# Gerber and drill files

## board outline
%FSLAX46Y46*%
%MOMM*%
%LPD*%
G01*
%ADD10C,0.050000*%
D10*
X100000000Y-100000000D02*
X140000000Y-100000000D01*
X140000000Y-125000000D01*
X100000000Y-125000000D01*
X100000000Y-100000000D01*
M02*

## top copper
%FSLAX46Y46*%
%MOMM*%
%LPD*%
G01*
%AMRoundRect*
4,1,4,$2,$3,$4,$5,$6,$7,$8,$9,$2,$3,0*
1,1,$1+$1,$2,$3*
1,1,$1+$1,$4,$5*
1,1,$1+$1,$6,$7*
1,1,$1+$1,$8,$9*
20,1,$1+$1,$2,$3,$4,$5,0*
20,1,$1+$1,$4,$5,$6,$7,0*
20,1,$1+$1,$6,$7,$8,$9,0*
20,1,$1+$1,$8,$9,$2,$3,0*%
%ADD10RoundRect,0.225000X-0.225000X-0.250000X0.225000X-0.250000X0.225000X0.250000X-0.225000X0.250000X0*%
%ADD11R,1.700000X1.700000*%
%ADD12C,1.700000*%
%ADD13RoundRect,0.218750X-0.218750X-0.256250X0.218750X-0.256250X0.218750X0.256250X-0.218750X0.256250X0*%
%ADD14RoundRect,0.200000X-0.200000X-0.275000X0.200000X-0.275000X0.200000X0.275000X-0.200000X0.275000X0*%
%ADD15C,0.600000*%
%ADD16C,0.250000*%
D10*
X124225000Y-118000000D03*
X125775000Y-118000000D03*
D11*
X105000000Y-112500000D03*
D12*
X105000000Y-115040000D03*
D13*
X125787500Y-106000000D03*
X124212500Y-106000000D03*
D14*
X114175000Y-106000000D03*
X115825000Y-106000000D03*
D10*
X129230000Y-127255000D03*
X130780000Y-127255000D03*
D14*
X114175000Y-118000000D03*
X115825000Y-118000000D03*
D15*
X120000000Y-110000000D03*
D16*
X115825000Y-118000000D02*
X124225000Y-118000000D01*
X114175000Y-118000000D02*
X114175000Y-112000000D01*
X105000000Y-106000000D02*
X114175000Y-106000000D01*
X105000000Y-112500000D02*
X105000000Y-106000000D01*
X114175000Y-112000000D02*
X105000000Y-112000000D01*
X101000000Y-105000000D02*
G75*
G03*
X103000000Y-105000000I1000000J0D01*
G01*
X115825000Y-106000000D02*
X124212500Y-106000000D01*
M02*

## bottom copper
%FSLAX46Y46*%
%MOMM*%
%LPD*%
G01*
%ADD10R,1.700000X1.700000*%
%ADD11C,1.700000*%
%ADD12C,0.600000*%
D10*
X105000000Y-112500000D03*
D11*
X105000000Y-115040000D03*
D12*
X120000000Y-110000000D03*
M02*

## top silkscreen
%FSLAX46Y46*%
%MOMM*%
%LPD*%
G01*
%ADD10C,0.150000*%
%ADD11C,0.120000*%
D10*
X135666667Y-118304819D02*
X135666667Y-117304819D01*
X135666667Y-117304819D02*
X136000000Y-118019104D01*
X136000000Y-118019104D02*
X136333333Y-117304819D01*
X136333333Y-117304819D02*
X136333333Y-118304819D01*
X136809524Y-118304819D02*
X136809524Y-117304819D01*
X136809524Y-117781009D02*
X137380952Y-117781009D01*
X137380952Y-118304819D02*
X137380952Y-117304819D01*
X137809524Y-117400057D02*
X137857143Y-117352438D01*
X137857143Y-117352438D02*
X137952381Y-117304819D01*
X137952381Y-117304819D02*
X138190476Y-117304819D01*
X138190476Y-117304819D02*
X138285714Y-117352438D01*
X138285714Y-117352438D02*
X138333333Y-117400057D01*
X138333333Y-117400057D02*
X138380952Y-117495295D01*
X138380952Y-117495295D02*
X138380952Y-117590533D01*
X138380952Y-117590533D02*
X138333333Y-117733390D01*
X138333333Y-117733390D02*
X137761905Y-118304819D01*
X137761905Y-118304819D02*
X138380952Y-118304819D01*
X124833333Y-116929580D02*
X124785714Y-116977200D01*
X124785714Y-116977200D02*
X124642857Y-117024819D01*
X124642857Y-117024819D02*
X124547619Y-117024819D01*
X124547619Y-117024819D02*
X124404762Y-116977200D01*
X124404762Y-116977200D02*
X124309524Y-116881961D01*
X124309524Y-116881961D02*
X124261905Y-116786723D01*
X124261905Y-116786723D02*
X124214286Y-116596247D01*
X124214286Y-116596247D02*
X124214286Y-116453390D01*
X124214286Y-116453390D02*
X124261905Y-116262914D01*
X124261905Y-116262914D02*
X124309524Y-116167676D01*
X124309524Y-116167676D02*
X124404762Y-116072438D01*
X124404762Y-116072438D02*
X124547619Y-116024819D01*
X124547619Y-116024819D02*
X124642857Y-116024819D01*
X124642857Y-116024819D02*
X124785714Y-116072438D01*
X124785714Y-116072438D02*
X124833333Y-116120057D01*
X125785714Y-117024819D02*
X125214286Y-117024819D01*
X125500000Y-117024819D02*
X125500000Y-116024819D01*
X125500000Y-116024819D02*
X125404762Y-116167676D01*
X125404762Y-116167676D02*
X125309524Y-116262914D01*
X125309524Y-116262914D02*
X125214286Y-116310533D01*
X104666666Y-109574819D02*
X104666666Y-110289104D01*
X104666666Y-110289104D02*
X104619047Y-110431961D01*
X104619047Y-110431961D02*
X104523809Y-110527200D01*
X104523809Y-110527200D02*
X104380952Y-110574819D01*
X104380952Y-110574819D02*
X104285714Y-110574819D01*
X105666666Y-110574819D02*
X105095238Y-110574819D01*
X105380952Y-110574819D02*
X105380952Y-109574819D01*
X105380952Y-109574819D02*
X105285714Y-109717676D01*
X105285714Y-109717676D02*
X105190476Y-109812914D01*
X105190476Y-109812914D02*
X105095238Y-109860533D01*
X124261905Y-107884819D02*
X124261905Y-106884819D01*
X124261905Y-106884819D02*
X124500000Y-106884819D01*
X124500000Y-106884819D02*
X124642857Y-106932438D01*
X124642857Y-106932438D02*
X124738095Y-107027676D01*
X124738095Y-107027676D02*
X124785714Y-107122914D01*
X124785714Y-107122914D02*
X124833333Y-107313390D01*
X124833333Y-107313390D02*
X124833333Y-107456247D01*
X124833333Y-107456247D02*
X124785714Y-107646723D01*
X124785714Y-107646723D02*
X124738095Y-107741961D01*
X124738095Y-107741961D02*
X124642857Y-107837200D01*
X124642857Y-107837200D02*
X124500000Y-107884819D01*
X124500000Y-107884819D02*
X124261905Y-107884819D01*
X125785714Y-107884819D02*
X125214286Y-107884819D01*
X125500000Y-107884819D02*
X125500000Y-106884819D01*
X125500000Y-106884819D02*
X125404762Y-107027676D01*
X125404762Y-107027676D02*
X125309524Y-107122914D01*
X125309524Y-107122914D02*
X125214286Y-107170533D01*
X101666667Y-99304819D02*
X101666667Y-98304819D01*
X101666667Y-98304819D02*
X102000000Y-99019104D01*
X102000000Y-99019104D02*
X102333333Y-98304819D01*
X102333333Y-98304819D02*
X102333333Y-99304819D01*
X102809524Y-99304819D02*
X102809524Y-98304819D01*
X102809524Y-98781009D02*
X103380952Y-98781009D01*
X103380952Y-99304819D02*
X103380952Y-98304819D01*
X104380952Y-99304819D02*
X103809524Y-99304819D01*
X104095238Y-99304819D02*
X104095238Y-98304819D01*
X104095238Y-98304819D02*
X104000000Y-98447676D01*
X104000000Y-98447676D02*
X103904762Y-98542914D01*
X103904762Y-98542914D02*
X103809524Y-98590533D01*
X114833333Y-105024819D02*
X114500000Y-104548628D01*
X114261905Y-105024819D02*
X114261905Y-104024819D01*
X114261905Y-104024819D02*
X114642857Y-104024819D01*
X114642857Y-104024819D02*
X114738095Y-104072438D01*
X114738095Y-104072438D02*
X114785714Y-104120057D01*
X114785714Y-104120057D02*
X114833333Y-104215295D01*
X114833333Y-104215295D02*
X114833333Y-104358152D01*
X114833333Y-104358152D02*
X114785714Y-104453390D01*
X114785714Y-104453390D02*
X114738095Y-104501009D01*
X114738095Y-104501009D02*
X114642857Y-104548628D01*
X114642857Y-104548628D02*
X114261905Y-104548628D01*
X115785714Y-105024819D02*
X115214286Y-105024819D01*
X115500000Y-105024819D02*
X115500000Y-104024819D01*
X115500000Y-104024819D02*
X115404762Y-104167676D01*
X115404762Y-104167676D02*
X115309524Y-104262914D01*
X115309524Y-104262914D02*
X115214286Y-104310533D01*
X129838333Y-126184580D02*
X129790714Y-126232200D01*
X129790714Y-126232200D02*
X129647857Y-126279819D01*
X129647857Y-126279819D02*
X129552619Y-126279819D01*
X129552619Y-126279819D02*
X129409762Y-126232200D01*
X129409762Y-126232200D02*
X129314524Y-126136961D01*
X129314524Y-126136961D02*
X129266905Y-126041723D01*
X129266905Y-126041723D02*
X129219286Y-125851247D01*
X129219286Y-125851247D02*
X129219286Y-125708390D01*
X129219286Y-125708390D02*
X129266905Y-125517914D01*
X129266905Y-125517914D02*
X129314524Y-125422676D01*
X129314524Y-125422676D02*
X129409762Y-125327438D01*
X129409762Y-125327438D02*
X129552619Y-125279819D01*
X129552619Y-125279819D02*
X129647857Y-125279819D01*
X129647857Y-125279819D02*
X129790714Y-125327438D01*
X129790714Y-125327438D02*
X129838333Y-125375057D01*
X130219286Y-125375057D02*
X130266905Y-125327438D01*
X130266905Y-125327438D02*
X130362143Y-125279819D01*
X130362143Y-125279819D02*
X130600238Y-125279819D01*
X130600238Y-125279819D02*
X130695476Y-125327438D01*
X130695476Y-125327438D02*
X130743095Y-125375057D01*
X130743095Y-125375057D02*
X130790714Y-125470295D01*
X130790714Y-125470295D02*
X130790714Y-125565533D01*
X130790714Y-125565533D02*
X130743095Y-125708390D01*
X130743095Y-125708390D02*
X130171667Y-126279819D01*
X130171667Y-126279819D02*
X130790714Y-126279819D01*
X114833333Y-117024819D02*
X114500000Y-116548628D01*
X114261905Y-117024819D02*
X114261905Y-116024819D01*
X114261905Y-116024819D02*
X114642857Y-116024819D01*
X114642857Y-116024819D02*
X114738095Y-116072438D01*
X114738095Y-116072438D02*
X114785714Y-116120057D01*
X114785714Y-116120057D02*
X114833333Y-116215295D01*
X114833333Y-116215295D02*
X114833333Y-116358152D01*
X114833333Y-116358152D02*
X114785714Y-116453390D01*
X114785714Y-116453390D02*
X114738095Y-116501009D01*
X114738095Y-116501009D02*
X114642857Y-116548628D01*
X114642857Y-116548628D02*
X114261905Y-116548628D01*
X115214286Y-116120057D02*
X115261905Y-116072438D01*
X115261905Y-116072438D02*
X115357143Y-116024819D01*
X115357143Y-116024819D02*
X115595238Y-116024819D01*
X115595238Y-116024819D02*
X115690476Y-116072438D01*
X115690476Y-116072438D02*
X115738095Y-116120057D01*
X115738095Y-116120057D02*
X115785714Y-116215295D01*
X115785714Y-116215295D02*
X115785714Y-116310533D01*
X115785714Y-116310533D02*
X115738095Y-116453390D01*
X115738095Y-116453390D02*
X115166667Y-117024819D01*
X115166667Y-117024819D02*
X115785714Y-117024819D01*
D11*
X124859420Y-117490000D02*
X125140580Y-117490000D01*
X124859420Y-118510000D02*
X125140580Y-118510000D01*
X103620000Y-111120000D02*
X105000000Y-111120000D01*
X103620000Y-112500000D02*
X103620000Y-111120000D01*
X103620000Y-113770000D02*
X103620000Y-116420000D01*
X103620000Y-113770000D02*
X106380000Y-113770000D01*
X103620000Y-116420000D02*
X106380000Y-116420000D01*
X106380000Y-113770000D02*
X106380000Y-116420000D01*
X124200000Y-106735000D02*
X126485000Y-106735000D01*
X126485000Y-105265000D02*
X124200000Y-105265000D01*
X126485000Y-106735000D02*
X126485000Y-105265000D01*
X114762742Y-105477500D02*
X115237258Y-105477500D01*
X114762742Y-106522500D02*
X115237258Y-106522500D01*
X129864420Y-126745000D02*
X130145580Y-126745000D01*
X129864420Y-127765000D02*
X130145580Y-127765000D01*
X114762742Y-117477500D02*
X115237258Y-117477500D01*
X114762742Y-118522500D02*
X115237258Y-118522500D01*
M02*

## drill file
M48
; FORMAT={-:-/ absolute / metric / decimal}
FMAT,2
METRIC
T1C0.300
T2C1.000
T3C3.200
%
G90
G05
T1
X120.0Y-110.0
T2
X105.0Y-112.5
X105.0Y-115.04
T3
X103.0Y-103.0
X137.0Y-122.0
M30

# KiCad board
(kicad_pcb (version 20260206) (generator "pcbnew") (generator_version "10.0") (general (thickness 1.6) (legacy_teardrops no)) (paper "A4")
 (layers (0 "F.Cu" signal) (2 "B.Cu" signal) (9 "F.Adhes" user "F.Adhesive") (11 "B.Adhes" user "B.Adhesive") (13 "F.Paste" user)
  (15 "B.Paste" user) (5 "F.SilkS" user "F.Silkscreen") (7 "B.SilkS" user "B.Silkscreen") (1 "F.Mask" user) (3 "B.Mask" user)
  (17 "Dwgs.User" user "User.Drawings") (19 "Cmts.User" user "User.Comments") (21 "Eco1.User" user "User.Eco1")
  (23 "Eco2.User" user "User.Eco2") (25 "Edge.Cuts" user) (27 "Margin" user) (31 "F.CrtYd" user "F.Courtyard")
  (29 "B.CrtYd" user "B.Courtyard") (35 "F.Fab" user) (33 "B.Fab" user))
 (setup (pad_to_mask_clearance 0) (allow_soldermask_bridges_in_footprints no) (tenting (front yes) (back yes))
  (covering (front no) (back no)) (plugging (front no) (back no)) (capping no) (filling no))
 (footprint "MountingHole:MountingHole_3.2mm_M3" (layer "F.Cu") (at 137 122)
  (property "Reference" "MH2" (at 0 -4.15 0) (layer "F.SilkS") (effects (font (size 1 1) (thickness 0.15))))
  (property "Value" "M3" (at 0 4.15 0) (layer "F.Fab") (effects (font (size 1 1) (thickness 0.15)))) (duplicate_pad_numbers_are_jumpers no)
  (pad "" np_thru_hole circle (at 0 0) (size 3.2 3.2) (drill 3.2) (layers "*.Cu" "*.Mask")))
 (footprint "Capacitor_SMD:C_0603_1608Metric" (layer "F.Cu") (at 125 118)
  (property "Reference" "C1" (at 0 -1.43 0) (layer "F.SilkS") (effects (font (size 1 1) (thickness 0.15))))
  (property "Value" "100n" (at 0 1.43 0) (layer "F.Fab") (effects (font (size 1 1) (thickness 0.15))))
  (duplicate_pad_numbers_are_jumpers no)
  (fp_line (start -0.14058 -0.51) (end 0.14058 -0.51) (stroke (width 0.12) (type solid)) (layer "F.SilkS"))
  (fp_line (start -0.14058 0.51) (end 0.14058 0.51) (stroke (width 0.12) (type solid)) (layer "F.SilkS"))
  (pad "1" smd roundrect (at -0.775 0) (size 0.9 0.95) (layers "F.Cu" "F.Mask" "F.Paste") (roundrect_rratio 0.25) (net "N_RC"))
  (pad "2" smd roundrect (at 0.775 0) (size 0.9 0.95) (layers "F.Cu" "F.Mask" "F.Paste") (roundrect_rratio 0.25) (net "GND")))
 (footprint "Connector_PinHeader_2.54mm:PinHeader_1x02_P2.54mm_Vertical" (layer "F.Cu") (at 105 112.5)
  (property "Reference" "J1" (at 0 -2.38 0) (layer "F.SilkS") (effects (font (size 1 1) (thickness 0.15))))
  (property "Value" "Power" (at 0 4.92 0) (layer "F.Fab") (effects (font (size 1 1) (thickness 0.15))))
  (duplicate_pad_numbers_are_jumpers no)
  (fp_line (start -1.38 -1.38) (end 0 -1.38) (stroke (width 0.12) (type solid)) (layer "F.SilkS"))
  (fp_line (start -1.38 0) (end -1.38 -1.38) (stroke (width 0.12) (type solid)) (layer "F.SilkS"))
  (fp_line (start -1.38 1.27) (end -1.38 3.92) (stroke (width 0.12) (type solid)) (layer "F.SilkS"))
  (fp_line (start -1.38 1.27) (end 1.38 1.27) (stroke (width 0.12) (type solid)) (layer "F.SilkS"))
  (fp_line (start -1.38 3.92) (end 1.38 3.92) (stroke (width 0.12) (type solid)) (layer "F.SilkS"))
  (fp_line (start 1.38 1.27) (end 1.38 3.92) (stroke (width 0.12) (type solid)) (layer "F.SilkS"))
  (pad "1" thru_hole rect (at 0 0) (size 1.7 1.7) (drill 1) (layers "*.Cu" "*.Mask") (remove_unused_layers no) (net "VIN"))
  (pad "2" thru_hole circle (at 0 2.54) (size 1.7 1.7) (drill 1) (layers "*.Cu" "*.Mask") (remove_unused_layers no) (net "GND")))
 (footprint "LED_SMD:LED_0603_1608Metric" (layer "F.Cu") (at 125 106 180)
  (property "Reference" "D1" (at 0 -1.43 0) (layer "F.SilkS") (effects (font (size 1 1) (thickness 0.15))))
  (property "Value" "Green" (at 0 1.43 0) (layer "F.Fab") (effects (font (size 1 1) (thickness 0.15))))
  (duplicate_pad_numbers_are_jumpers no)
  (fp_line (start 0.8 -0.735) (end -1.485 -0.735) (stroke (width 0.12) (type solid)) (layer "F.SilkS"))
  (fp_line (start -1.485 0.735) (end 0.8 0.735) (stroke (width 0.12) (type solid)) (layer "F.SilkS"))
  (fp_line (start -1.485 -0.735) (end -1.485 0.735) (stroke (width 0.12) (type solid)) (layer "F.SilkS"))
  (pad "1" smd roundrect (at -0.7875 0) (size 0.875 0.95) (layers "F.Cu" "F.Mask" "F.Paste") (roundrect_rratio 0.25) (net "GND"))
  (pad "2" smd roundrect (at 0.7875 0) (size 0.875 0.95) (layers "F.Cu" "F.Mask" "F.Paste") (roundrect_rratio 0.25) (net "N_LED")))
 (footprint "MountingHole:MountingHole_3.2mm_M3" (layer "F.Cu") (at 103 103)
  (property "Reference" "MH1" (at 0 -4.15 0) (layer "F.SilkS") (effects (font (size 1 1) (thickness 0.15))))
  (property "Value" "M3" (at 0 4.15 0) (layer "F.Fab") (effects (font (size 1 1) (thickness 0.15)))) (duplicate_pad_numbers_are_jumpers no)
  (pad "" np_thru_hole circle (at 0 0) (size 3.2 3.2) (drill 3.2) (layers "*.Cu" "*.Mask")))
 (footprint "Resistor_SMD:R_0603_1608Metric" (layer "F.Cu") (at 115 106)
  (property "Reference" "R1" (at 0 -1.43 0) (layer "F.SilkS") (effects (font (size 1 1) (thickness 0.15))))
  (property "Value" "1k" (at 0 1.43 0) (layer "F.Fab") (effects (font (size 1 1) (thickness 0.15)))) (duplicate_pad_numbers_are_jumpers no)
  (fp_line (start -0.237258 -0.5225) (end 0.237258 -0.5225) (stroke (width 0.12) (type solid)) (layer "F.SilkS"))
  (fp_line (start -0.237258 0.5225) (end 0.237258 0.5225) (stroke (width 0.12) (type solid)) (layer "F.SilkS"))
  (pad "1" smd roundrect (at -0.825 0) (size 0.8 0.95) (layers "F.Cu" "F.Mask" "F.Paste") (roundrect_rratio 0.25) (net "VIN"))
  (pad "2" smd roundrect (at 0.825 0) (size 0.8 0.95) (layers "F.Cu" "F.Mask" "F.Paste") (roundrect_rratio 0.25) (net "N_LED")))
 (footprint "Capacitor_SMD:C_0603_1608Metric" (layer "F.Cu") (at 130.005 127.255)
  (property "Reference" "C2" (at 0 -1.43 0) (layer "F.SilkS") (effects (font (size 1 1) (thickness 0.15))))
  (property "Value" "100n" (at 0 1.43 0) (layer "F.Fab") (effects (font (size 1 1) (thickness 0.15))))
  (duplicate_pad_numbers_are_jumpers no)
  (fp_line (start -0.14058 -0.51) (end 0.14058 -0.51) (stroke (width 0.12) (type solid)) (layer "F.SilkS"))
  (fp_line (start -0.14058 0.51) (end 0.14058 0.51) (stroke (width 0.12) (type solid)) (layer "F.SilkS"))
  (pad "1" smd roundrect (at -0.775 0) (size 0.9 0.95) (layers "F.Cu" "F.Mask" "F.Paste") (roundrect_rratio 0.25) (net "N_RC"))
  (pad "2" smd roundrect (at 0.775 0) (size 0.9 0.95) (layers "F.Cu" "F.Mask" "F.Paste") (roundrect_rratio 0.25) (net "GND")))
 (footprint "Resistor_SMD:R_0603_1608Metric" (layer "F.Cu") (at 115 118)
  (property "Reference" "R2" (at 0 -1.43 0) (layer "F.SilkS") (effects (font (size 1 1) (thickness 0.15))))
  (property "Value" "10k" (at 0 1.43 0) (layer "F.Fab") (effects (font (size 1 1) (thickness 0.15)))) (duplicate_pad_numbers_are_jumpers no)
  (fp_line (start -0.237258 -0.5225) (end 0.237258 -0.5225) (stroke (width 0.12) (type solid)) (layer "F.SilkS"))
  (fp_line (start -0.237258 0.5225) (end 0.237258 0.5225) (stroke (width 0.12) (type solid)) (layer "F.SilkS"))
  (pad "1" smd roundrect (at -0.825 0) (size 0.8 0.95) (layers "F.Cu" "F.Mask" "F.Paste") (roundrect_rratio 0.25) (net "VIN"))
  (pad "2" smd roundrect (at 0.825 0) (size 0.8 0.95) (layers "F.Cu" "F.Mask" "F.Paste") (roundrect_rratio 0.25) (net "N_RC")))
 (gr_rect (start 100 100) (end 140 125) (stroke (width 0.05) (type default)) (fill no) (layer "Edge.Cuts"))
 (segment (start 115.825 118) (end 124.225 118) (width 0.25) (layer "F.Cu") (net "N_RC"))
 (segment (start 114.175 118) (end 114.175 112) (width 0.25) (layer "F.Cu") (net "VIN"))
 (segment (start 105 106) (end 114.175 106) (width 0.25) (layer "F.Cu") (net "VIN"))
 (segment (start 105 112.5) (end 105 106) (width 0.25) (layer "F.Cu") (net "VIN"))
 (segment (start 114.175 112) (end 105 112) (width 0.25) (layer "F.Cu") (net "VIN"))
 (via (at 120 110) (size 0.6) (drill 0.3) (layers "F.Cu" "B.Cu") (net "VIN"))
 (arc (start 101 105) (mid 102 106) (end 103 105) (width 0.25) (layer "F.Cu") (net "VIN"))
 (segment (start 115.825 106) (end 124.2125 106) (width 0.25) (layer "F.Cu") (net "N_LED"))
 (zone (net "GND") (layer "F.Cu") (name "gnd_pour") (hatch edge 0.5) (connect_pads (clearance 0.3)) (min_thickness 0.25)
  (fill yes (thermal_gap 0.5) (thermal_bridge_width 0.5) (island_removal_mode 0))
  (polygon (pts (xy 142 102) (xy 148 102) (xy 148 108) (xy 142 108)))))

